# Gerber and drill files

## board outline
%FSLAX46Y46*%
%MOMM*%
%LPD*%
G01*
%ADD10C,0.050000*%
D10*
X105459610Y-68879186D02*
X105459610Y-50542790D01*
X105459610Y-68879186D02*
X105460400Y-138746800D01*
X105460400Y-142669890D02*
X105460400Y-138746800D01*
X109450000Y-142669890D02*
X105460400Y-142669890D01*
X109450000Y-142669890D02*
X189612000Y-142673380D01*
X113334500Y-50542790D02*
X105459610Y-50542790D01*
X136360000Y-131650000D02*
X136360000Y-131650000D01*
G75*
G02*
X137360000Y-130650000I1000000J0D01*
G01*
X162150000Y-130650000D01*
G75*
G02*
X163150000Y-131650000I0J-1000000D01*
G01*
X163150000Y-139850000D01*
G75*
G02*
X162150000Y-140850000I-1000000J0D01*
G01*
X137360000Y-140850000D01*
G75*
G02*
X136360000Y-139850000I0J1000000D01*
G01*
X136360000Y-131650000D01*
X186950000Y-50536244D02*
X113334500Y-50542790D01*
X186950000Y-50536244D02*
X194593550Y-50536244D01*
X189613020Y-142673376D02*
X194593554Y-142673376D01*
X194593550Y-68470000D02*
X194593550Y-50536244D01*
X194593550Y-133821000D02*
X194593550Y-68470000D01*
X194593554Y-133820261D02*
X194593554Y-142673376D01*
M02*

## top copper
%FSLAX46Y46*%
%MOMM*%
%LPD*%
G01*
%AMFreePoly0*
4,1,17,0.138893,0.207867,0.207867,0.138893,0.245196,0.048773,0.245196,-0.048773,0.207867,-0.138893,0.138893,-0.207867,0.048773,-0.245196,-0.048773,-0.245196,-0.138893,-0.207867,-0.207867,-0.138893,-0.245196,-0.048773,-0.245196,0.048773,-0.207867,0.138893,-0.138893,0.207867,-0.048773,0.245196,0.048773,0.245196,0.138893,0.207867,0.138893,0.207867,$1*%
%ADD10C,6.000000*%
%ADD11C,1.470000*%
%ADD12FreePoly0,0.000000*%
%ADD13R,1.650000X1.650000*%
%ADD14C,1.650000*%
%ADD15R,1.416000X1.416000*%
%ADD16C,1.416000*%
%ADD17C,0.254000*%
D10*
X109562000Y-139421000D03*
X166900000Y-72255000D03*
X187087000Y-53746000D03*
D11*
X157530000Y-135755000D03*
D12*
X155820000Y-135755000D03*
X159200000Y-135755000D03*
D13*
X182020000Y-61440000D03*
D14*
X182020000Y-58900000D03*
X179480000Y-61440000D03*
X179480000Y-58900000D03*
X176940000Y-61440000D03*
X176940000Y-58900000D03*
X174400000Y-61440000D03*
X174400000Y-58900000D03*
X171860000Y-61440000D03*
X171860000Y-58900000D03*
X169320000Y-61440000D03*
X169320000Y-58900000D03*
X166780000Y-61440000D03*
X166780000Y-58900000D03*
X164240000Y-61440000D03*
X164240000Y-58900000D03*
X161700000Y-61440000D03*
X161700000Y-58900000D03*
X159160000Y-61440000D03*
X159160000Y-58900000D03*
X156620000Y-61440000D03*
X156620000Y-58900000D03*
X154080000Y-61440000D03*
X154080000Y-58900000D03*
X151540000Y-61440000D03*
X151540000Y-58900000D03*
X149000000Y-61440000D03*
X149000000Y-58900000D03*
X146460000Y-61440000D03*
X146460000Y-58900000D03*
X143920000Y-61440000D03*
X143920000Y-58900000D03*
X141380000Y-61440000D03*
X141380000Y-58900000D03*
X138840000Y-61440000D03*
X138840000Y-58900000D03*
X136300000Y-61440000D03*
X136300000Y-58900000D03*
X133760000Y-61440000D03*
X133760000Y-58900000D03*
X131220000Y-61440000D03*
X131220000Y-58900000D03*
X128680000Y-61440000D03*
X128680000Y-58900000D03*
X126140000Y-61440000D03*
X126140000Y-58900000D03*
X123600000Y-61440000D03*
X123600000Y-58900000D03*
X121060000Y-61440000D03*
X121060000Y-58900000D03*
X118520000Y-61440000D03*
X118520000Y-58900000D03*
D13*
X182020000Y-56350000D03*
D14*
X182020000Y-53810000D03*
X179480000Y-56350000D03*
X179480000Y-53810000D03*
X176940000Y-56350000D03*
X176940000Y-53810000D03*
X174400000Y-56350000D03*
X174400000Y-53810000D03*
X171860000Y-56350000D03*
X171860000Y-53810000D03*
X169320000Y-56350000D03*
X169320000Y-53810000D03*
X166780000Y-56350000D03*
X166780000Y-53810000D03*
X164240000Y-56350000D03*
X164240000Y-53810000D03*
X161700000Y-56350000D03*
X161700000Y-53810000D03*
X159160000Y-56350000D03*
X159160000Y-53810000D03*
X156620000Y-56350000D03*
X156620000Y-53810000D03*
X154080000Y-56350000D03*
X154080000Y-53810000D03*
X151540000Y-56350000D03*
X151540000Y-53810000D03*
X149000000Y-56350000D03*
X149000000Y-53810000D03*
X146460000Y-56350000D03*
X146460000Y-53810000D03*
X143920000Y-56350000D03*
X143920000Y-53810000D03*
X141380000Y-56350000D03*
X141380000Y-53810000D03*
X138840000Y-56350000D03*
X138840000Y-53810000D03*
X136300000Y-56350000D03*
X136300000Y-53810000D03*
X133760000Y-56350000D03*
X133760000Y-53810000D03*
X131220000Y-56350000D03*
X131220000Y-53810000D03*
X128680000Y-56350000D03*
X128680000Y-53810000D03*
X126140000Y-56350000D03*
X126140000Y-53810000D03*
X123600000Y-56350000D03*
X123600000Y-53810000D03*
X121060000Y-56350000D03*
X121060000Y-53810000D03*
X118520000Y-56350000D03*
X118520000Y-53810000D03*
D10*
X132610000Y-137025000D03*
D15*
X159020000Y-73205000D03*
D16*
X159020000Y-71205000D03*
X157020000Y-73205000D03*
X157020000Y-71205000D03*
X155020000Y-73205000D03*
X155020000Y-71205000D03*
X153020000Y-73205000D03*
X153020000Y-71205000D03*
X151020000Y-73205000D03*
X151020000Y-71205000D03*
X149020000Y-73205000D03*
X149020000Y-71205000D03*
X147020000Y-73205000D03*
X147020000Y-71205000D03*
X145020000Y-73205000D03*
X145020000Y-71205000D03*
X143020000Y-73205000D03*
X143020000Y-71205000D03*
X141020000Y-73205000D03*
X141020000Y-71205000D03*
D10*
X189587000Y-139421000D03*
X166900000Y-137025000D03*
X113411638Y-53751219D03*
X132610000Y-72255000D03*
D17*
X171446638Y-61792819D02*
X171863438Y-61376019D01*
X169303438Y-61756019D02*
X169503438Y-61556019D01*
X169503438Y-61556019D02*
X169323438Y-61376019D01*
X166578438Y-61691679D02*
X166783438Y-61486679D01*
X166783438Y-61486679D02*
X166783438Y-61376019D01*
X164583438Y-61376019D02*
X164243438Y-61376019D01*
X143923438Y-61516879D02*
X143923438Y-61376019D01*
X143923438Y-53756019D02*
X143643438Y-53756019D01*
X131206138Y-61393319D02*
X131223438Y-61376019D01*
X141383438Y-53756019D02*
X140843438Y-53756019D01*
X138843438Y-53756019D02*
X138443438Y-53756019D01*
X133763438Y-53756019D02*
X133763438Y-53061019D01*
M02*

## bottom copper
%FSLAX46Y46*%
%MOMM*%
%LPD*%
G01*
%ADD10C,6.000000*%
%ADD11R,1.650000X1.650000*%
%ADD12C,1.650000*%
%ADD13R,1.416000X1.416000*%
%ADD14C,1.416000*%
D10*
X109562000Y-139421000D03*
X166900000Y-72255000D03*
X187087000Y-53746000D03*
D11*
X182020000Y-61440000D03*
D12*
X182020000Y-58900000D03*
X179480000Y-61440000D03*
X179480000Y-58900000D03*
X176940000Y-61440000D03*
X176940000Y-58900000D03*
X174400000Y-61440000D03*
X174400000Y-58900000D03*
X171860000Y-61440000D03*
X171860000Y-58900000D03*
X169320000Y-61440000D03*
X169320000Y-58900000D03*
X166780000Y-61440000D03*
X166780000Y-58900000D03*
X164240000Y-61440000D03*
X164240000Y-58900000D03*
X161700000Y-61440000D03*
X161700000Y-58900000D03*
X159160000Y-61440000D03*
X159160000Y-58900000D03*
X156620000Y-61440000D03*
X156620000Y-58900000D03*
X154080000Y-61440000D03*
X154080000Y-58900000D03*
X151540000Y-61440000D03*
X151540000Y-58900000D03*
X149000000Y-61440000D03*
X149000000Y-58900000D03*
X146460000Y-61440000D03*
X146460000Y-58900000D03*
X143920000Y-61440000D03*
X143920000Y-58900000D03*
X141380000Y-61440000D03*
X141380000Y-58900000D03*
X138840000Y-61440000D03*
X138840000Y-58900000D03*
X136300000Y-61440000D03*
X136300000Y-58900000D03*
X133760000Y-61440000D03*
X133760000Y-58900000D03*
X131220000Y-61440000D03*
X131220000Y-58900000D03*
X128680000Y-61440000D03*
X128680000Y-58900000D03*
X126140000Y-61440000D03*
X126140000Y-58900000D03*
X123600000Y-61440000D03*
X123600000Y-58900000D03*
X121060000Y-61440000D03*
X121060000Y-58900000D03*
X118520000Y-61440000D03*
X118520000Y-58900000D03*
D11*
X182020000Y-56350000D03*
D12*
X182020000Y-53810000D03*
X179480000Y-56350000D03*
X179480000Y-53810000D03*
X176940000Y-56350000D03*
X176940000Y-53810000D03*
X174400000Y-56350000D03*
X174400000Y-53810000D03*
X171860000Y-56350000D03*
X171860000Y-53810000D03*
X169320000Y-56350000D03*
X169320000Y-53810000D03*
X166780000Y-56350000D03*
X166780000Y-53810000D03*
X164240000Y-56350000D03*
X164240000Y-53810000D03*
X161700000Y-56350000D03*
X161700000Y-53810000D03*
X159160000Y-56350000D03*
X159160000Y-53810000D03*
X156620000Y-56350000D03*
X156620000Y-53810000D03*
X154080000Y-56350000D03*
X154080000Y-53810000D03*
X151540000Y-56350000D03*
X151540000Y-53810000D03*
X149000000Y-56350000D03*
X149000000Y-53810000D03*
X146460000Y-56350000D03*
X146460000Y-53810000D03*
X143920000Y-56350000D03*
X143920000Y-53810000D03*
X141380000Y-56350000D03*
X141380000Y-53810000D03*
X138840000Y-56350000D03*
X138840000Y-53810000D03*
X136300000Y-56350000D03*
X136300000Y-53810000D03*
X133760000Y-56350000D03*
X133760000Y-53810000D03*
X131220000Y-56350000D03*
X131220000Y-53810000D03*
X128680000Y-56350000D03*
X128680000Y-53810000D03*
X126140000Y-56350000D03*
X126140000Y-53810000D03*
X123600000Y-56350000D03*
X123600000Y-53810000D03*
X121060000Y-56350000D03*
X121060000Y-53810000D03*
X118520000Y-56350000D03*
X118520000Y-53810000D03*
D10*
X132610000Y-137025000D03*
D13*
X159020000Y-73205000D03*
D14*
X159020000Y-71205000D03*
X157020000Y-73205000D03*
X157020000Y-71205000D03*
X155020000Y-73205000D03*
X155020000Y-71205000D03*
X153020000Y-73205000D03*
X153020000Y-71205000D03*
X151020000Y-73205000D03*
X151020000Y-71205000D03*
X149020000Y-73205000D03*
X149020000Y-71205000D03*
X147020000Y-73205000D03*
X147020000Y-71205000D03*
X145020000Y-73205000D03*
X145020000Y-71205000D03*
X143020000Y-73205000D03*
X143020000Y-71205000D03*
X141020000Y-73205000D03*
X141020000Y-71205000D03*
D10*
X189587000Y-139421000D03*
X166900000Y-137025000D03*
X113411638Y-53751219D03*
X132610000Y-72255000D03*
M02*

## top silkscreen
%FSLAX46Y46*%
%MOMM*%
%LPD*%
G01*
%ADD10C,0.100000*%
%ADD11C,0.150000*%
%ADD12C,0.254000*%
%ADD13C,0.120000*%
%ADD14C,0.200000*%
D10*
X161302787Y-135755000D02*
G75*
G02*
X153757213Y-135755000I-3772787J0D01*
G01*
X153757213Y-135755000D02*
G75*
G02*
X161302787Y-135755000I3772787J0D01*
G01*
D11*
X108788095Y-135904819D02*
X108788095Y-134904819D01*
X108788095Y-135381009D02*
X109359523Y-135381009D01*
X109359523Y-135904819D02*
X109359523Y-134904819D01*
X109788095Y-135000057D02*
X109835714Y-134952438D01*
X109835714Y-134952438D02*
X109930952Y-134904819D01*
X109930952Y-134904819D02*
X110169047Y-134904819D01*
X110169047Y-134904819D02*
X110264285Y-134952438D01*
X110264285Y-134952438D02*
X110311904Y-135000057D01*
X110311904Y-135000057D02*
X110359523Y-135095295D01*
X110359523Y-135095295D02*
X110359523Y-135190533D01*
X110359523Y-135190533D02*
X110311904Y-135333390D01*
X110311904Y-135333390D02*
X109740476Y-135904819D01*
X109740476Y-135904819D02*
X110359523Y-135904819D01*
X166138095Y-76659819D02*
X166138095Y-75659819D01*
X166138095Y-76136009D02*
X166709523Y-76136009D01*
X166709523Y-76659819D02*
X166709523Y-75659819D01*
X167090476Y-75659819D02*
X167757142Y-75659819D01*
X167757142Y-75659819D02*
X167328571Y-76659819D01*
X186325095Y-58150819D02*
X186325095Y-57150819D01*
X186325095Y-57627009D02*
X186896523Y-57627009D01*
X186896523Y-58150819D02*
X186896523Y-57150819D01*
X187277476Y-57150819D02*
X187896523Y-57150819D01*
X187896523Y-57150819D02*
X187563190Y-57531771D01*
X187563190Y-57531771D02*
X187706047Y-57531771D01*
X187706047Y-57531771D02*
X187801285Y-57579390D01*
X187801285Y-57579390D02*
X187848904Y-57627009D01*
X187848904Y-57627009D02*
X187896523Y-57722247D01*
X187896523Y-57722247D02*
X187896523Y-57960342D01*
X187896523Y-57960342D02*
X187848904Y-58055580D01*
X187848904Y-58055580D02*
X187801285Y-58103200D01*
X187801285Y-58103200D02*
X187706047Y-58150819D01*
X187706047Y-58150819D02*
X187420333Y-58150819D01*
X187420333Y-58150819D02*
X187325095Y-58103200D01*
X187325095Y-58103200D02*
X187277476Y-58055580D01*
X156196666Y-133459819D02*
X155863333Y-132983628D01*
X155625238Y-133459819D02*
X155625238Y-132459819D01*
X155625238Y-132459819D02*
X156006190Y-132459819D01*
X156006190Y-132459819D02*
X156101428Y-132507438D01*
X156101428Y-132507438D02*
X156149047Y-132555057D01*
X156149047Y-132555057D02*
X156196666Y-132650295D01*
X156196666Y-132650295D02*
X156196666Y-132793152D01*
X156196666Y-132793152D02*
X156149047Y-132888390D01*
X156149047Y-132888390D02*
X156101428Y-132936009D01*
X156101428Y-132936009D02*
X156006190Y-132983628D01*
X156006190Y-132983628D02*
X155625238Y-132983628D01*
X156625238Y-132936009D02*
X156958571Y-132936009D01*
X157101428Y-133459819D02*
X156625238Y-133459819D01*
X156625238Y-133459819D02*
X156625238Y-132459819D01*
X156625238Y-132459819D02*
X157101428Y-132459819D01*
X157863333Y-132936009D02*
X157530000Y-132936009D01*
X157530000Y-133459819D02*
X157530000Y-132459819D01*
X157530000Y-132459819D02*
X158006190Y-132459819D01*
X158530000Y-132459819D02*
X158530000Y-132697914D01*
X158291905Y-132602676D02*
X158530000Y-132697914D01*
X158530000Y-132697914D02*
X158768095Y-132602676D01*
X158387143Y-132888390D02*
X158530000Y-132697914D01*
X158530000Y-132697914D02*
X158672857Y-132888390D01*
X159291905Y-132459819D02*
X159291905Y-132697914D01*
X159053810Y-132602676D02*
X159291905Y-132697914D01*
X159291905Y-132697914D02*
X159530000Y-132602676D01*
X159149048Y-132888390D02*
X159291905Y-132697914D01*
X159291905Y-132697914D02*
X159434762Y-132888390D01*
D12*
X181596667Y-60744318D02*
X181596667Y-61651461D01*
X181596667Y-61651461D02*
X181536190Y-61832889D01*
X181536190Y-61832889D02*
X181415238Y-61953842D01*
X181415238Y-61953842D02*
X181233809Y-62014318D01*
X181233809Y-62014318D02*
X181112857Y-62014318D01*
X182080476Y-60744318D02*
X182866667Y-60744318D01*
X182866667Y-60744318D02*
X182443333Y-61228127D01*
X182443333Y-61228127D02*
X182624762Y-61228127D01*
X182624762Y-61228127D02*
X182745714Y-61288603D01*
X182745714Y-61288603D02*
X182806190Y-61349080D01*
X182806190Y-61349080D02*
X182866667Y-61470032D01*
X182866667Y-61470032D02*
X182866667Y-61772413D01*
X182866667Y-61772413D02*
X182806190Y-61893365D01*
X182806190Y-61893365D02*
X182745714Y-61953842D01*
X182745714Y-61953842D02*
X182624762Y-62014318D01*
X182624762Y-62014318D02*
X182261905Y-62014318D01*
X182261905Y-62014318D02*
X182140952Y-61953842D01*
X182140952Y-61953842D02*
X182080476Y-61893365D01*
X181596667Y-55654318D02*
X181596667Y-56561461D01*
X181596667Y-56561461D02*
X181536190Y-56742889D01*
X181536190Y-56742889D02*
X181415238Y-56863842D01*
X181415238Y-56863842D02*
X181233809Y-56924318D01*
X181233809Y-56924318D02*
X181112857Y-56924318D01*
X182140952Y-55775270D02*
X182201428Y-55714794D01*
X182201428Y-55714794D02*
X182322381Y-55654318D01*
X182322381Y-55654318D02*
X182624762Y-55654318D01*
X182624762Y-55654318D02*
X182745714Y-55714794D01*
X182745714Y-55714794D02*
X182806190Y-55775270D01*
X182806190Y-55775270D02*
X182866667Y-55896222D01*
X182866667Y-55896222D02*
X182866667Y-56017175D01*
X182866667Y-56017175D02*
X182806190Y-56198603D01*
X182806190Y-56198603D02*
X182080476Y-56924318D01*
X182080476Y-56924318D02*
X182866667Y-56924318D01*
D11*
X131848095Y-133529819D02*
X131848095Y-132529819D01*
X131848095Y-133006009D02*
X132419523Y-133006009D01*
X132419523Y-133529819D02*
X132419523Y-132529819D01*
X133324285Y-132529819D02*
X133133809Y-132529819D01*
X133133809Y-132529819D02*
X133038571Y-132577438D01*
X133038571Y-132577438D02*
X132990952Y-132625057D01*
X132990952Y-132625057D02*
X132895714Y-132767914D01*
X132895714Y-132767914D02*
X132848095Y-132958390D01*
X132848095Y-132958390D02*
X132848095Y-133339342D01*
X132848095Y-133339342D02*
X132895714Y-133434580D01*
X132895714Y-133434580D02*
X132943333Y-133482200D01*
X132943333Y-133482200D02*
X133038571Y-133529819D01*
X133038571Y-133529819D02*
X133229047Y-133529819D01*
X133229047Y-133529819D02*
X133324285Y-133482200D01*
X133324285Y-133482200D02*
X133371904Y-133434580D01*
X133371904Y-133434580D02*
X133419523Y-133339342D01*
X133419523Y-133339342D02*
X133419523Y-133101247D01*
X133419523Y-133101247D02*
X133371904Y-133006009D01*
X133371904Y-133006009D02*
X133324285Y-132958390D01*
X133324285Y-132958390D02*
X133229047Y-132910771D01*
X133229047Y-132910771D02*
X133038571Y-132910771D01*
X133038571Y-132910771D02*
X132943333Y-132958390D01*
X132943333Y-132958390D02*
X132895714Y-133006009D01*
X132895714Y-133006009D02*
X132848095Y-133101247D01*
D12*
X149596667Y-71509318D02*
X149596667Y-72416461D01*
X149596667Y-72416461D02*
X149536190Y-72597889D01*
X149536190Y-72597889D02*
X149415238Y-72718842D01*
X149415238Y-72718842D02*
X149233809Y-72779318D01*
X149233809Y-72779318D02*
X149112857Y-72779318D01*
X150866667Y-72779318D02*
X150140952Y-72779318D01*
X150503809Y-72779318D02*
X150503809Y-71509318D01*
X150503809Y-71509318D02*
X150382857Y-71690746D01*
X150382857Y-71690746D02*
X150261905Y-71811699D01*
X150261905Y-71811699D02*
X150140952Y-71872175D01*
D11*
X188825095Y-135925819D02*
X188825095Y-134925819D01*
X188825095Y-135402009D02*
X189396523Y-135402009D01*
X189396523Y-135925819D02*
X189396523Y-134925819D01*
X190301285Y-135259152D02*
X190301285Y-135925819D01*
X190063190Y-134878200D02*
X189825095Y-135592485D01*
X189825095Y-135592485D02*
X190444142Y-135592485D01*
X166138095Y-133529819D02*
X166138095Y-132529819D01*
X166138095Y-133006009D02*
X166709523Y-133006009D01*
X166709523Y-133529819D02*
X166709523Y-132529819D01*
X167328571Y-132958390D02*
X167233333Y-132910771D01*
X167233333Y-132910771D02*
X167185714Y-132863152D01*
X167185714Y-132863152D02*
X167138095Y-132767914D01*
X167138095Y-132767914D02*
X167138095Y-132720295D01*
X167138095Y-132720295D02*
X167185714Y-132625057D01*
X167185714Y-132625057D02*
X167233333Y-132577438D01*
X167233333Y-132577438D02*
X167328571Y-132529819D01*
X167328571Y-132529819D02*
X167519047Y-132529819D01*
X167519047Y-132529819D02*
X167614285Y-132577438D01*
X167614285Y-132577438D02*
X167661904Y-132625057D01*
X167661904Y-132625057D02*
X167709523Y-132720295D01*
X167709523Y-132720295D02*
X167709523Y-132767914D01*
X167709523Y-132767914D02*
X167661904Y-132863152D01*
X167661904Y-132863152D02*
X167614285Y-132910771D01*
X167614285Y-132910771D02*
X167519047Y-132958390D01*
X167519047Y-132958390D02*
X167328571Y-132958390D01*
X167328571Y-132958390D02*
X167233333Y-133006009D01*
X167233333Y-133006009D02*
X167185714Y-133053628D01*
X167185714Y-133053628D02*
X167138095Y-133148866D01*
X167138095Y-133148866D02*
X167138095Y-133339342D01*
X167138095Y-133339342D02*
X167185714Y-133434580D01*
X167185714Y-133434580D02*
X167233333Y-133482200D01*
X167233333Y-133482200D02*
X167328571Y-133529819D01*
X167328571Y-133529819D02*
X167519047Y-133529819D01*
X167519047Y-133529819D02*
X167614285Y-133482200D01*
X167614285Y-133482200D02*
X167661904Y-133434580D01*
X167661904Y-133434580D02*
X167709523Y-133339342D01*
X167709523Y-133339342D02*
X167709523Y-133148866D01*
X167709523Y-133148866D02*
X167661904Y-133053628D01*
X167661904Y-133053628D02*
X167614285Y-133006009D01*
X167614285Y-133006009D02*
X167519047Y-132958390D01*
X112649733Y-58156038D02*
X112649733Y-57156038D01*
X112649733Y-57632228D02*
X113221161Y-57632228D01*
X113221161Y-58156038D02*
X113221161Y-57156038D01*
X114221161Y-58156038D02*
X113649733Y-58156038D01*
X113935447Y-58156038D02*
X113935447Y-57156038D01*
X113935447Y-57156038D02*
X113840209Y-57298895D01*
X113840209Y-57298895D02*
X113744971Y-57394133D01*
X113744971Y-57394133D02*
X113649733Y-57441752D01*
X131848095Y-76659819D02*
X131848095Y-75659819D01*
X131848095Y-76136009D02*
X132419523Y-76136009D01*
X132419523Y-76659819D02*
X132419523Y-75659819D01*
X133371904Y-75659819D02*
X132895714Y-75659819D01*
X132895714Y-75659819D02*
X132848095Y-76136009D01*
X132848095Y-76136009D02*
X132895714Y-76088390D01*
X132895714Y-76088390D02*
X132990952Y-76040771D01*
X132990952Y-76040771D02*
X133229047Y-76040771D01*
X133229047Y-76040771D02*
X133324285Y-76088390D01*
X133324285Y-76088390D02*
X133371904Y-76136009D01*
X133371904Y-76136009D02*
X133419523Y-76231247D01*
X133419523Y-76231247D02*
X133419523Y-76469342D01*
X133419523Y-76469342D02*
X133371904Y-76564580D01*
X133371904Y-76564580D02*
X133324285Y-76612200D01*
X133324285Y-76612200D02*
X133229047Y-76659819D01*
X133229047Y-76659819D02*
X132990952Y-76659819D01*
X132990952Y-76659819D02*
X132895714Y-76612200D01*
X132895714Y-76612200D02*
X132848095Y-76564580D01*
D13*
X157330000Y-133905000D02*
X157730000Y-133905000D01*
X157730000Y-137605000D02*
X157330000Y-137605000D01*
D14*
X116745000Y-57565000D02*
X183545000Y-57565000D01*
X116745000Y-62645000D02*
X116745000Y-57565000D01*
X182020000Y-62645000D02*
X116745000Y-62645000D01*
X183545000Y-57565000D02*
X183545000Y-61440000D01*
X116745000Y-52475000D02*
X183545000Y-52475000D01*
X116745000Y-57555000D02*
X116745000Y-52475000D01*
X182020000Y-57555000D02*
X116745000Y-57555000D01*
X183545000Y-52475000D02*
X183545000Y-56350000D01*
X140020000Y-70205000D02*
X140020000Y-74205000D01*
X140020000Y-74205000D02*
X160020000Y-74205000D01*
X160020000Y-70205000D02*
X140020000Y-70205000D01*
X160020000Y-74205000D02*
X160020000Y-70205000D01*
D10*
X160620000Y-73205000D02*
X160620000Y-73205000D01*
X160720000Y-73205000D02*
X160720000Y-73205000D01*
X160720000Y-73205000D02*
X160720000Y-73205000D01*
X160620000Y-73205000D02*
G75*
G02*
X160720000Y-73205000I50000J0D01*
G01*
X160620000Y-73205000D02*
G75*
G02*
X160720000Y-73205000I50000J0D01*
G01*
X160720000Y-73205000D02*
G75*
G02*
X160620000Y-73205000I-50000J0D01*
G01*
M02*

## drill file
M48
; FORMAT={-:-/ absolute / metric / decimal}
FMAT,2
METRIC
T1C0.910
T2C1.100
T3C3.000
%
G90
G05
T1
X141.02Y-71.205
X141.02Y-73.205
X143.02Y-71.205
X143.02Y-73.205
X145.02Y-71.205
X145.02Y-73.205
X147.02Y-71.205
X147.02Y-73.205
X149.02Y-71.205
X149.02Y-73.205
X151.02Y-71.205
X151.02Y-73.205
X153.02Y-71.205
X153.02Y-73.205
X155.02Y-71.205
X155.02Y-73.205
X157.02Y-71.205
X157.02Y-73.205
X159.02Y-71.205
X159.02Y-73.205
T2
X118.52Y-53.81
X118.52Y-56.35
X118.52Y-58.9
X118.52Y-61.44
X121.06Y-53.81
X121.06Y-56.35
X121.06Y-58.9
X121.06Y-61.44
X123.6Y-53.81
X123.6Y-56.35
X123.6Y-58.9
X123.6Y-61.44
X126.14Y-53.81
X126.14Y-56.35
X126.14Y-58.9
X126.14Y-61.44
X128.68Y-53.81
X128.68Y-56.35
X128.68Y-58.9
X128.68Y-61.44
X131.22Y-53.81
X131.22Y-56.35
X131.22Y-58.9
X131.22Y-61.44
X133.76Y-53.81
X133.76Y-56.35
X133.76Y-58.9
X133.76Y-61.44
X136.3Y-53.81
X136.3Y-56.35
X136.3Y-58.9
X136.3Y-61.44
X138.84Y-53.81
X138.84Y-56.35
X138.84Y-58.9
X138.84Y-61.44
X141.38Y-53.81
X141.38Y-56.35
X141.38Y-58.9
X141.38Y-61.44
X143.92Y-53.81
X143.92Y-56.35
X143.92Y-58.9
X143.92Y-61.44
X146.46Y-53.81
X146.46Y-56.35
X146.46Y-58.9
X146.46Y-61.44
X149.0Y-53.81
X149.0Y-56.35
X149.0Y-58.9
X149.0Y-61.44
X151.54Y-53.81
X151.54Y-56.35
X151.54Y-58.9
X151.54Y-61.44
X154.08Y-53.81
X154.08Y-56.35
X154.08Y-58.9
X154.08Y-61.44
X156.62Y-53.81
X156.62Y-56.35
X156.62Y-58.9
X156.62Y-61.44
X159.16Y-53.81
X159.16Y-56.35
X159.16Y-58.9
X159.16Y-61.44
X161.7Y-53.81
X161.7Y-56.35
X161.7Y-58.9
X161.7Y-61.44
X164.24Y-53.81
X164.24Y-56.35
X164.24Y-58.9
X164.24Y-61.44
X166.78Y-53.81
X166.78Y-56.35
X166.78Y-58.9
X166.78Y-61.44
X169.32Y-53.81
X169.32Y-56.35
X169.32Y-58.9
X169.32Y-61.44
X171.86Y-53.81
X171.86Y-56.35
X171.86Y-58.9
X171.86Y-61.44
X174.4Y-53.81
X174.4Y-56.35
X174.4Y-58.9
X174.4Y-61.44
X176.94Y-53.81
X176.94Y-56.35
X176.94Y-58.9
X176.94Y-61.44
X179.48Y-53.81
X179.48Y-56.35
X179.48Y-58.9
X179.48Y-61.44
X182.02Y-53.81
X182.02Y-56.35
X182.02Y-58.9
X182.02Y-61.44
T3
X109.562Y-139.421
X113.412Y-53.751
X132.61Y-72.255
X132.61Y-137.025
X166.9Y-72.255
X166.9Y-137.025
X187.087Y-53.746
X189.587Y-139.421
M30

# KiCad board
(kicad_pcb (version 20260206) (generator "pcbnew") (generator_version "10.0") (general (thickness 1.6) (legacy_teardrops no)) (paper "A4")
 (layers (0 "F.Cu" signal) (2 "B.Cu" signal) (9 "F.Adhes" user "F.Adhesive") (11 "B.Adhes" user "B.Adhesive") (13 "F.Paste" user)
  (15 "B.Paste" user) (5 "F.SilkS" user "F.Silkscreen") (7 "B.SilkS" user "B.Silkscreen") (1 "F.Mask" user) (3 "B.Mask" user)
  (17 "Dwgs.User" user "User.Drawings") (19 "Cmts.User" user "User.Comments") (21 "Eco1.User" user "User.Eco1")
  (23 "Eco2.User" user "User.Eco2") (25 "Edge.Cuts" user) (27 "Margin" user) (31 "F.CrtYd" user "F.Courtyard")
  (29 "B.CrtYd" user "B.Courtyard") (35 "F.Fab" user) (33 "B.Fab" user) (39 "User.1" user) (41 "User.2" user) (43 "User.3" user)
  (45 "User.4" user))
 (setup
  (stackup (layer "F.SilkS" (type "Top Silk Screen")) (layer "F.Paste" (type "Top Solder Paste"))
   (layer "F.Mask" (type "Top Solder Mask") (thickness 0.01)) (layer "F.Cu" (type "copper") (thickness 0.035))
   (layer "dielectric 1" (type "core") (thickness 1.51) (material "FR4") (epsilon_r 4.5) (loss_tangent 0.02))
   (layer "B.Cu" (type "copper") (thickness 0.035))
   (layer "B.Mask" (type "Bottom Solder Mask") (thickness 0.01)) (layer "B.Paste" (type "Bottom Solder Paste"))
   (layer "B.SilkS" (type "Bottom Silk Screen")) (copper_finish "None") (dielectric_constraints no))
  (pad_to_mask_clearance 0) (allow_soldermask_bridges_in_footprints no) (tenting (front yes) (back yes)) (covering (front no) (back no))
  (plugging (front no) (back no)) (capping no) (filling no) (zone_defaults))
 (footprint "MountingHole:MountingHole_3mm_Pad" (layer "F.Cu") (at 109.562 139.421 180)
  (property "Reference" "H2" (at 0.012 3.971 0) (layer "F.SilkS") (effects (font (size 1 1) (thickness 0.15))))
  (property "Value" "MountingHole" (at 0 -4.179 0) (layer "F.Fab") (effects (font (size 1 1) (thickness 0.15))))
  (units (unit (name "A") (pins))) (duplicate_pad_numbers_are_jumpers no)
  (pad "1" thru_hole circle (at 0 0 180) (size 6 6) (drill 3) (layers "*.Cu" "*.Mask") (remove_unused_layers no) (zone_connect 2)))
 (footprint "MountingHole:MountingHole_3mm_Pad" (layer "F.Cu") (at 166.9 72.255)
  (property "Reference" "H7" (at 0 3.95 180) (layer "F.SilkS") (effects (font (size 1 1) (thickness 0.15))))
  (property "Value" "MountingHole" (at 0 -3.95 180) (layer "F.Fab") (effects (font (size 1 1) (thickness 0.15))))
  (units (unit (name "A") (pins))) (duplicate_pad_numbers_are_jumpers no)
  (pad "1" thru_hole circle (at 0 0) (size 6 6) (drill 3) (layers "*.Cu" "*.Mask") (remove_unused_layers no) (zone_connect 2)))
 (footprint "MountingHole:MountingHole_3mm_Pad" (layer "F.Cu") (at 187.087 53.746 180)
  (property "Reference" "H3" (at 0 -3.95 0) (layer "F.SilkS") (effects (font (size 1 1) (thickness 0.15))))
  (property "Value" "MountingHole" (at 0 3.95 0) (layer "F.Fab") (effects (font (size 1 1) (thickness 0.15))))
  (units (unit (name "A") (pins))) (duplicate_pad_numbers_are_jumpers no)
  (pad "1" thru_hole circle (at 0 0 180) (size 6 6) (drill 3) (layers "*.Cu" "*.Mask") (remove_unused_layers no) (zone_connect 2)))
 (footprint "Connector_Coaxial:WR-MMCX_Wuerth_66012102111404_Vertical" (layer "F.Cu") (at 157.53 135.755)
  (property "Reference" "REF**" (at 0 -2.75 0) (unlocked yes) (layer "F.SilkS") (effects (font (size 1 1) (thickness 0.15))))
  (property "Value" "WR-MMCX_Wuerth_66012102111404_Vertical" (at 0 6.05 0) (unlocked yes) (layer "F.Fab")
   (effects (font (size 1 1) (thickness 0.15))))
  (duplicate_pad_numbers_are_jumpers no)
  (fp_line (start -0.2 -1.85) (end 0.2 -1.85) (stroke (width 0.12) (type solid)) (layer "F.SilkS"))
  (fp_line (start 0.2 1.85) (end -0.2 1.85) (stroke (width 0.12) (type solid)) (layer "F.SilkS"))
  (pad "1" smd circle (at 0 0) (size 1.47 1.47) (layers "F.Cu" "F.Mask" "F.Paste"))
  (pad "2" smd custom (at -1.71 0) (size 0.5 0.5) (layers "F.Cu" "F.Mask") (options (clearance outline) (anchor circle)) (primitives))
  (pad "2" smd custom (at 1.67 0) (size 0.5 0.5) (layers "F.Cu" "F.Mask") (options (clearance outline) (anchor circle)) (primitives)))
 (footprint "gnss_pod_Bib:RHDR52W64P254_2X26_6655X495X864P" (layer "F.Cu") (at 182.02 61.44)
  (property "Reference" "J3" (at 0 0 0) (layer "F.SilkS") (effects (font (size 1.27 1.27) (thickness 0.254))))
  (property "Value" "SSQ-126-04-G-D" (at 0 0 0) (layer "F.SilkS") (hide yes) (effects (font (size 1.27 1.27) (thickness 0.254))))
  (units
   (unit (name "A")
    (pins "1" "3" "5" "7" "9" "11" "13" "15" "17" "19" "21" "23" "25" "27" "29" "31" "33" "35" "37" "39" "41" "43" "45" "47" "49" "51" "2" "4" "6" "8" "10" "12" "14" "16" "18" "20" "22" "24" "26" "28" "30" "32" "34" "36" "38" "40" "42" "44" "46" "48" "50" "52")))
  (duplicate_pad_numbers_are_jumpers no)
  (fp_line (start -65.275 -3.875) (end 1.525 -3.875) (stroke (width 0.2) (type solid)) (layer "F.SilkS"))
  (fp_line (start -65.275 1.205) (end -65.275 -3.875) (stroke (width 0.2) (type solid)) (layer "F.SilkS"))
  (fp_line (start 0 1.205) (end -65.275 1.205) (stroke (width 0.2) (type solid)) (layer "F.SilkS"))
  (fp_line (start 1.525 -3.875) (end 1.525 0) (stroke (width 0.2) (type solid)) (layer "F.SilkS"))
  (pad "1" thru_hole rect (at 0 0) (size 1.65 1.65) (drill 1.1) (layers "*.Cu" "*.Mask") (remove_unused_layers no)
   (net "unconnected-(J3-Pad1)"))
  (pad "2" thru_hole circle (at 0 -2.54) (size 1.65 1.65) (drill 1.1) (layers "*.Cu" "*.Mask") (remove_unused_layers no)
   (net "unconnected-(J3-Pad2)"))
  (pad "3" thru_hole circle (at -2.54 0) (size 1.65 1.65) (drill 1.1) (layers "*.Cu" "*.Mask") (remove_unused_layers no)
   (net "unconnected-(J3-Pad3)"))
  (pad "4" thru_hole circle (at -2.54 -2.54) (size 1.65 1.65) (drill 1.1) (layers "*.Cu" "*.Mask") (remove_unused_layers no)
   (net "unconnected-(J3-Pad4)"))
  (pad "5" thru_hole circle (at -5.08 0) (size 1.65 1.65) (drill 1.1) (layers "*.Cu" "*.Mask") (remove_unused_layers no)
   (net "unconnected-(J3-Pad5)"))
  (pad "6" thru_hole circle (at -5.08 -2.54) (size 1.65 1.65) (drill 1.1) (layers "*.Cu" "*.Mask") (remove_unused_layers no)
   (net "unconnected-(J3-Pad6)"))
  (pad "7" thru_hole circle (at -7.62 0) (size 1.65 1.65) (drill 1.1) (layers "*.Cu" "*.Mask") (remove_unused_layers no)
   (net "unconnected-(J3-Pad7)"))
  (pad "8" thru_hole circle (at -7.62 -2.54) (size 1.65 1.65) (drill 1.1) (layers "*.Cu" "*.Mask") (remove_unused_layers no)
   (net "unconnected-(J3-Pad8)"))
  (pad "9" thru_hole circle (at -10.16 0) (size 1.65 1.65) (drill 1.1) (layers "*.Cu" "*.Mask") (remove_unused_layers no)
   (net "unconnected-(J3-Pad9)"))
  (pad "10" thru_hole circle (at -10.16 -2.54) (size 1.65 1.65) (drill 1.1) (layers "*.Cu" "*.Mask") (remove_unused_layers no)
   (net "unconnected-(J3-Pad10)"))
  (pad "11" thru_hole circle (at -12.7 0) (size 1.65 1.65) (drill 1.1) (layers "*.Cu" "*.Mask") (remove_unused_layers no)
   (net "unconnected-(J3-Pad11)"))
  (pad "12" thru_hole circle (at -12.7 -2.54) (size 1.65 1.65) (drill 1.1) (layers "*.Cu" "*.Mask") (remove_unused_layers no)
   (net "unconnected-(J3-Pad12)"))
  (pad "13" thru_hole circle (at -15.24 0) (size 1.65 1.65) (drill 1.1) (layers "*.Cu" "*.Mask") (remove_unused_layers no)
   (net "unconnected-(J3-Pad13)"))
  (pad "14" thru_hole circle (at -15.24 -2.54) (size 1.65 1.65) (drill 1.1) (layers "*.Cu" "*.Mask") (remove_unused_layers no)
   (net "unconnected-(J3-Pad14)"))
  (pad "15" thru_hole circle (at -17.78 0) (size 1.65 1.65) (drill 1.1) (layers "*.Cu" "*.Mask") (remove_unused_layers no)
   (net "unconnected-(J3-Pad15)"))
  (pad "16" thru_hole circle (at -17.78 -2.54) (size 1.65 1.65) (drill 1.1) (layers "*.Cu" "*.Mask") (remove_unused_layers no)
   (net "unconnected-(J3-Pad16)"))
  (pad "17" thru_hole circle (at -20.32 0) (size 1.65 1.65) (drill 1.1) (layers "*.Cu" "*.Mask") (remove_unused_layers no)
   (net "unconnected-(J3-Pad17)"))
  (pad "18" thru_hole circle (at -20.32 -2.54) (size 1.65 1.65) (drill 1.1) (layers "*.Cu" "*.Mask") (remove_unused_layers no)
   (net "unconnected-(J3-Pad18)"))
  (pad "19" thru_hole circle (at -22.86 0) (size 1.65 1.65) (drill 1.1) (layers "*.Cu" "*.Mask") (remove_unused_layers no)
   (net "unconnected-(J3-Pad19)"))
  (pad "20" thru_hole circle (at -22.86 -2.54) (size 1.65 1.65) (drill 1.1) (layers "*.Cu" "*.Mask") (remove_unused_layers no)
   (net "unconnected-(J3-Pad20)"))
  (pad "21" thru_hole circle (at -25.4 0) (size 1.65 1.65) (drill 1.1) (layers "*.Cu" "*.Mask") (remove_unused_layers no)
   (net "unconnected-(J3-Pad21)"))
  (pad "22" thru_hole circle (at -25.4 -2.54) (size 1.65 1.65) (drill 1.1) (layers "*.Cu" "*.Mask") (remove_unused_layers no)
   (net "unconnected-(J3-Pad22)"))
  (pad "23" thru_hole circle (at -27.94 0) (size 1.65 1.65) (drill 1.1) (layers "*.Cu" "*.Mask") (remove_unused_layers no)
   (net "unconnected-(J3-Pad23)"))
  (pad "24" thru_hole circle (at -27.94 -2.54) (size 1.65 1.65) (drill 1.1) (layers "*.Cu" "*.Mask") (remove_unused_layers no)
   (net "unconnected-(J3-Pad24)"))
  (pad "25" thru_hole circle (at -30.48 0) (size 1.65 1.65) (drill 1.1) (layers "*.Cu" "*.Mask") (remove_unused_layers no)
   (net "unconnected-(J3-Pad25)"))
  (pad "26" thru_hole circle (at -30.48 -2.54) (size 1.65 1.65) (drill 1.1) (layers "*.Cu" "*.Mask") (remove_unused_layers no)
   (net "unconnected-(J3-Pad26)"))
  (pad "27" thru_hole circle (at -33.02 0) (size 1.65 1.65) (drill 1.1) (layers "*.Cu" "*.Mask") (remove_unused_layers no)
   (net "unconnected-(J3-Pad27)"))
  (pad "28" thru_hole circle (at -33.02 -2.54) (size 1.65 1.65) (drill 1.1) (layers "*.Cu" "*.Mask") (remove_unused_layers no)
   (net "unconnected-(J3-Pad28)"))
  (pad "29" thru_hole circle (at -35.56 0) (size 1.65 1.65) (drill 1.1) (layers "*.Cu" "*.Mask") (remove_unused_layers no) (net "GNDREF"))
  (pad "30" thru_hole circle (at -35.56 -2.54) (size 1.65 1.65) (drill 1.1) (layers "*.Cu" "*.Mask") (remove_unused_layers no)
   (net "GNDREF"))
  (pad "31" thru_hole circle (at -38.1 0) (size 1.65 1.65) (drill 1.1) (layers "*.Cu" "*.Mask") (remove_unused_layers no) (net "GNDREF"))
  (pad "32" thru_hole circle (at -38.1 -2.54) (size 1.65 1.65) (drill 1.1) (layers "*.Cu" "*.Mask") (remove_unused_layers no) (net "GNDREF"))
  (pad "33" thru_hole circle (at -40.64 0) (size 1.65 1.65) (drill 1.1) (layers "*.Cu" "*.Mask") (remove_unused_layers no)
   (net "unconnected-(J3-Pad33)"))
  (pad "34" thru_hole circle (at -40.64 -2.54) (size 1.65 1.65) (drill 1.1) (layers "*.Cu" "*.Mask") (remove_unused_layers no)
   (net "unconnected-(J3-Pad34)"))
  (pad "35" thru_hole circle (at -43.18 0) (size 1.65 1.65) (drill 1.1) (layers "*.Cu" "*.Mask") (remove_unused_layers no)
   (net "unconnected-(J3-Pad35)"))
  (pad "36" thru_hole circle (at -43.18 -2.54) (size 1.65 1.65) (drill 1.1) (layers "*.Cu" "*.Mask") (remove_unused_layers no)
   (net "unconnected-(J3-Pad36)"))
  (pad "37" thru_hole circle (at -45.72 0) (size 1.65 1.65) (drill 1.1) (layers "*.Cu" "*.Mask") (remove_unused_layers no)
   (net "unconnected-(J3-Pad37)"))
  (pad "38" thru_hole circle (at -45.72 -2.54) (size 1.65 1.65) (drill 1.1) (layers "*.Cu" "*.Mask") (remove_unused_layers no)
   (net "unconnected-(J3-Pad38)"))
  (pad "39" thru_hole circle (at -48.26 0) (size 1.65 1.65) (drill 1.1) (layers "*.Cu" "*.Mask") (remove_unused_layers no)
   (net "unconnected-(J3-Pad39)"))
  (pad "40" thru_hole circle (at -48.26 -2.54) (size 1.65 1.65) (drill 1.1) (layers "*.Cu" "*.Mask") (remove_unused_layers no)
   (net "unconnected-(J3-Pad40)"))
  (pad "41" thru_hole circle (at -50.8 0) (size 1.65 1.65) (drill 1.1) (layers "*.Cu" "*.Mask") (remove_unused_layers no)
   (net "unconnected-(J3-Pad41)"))
  (pad "42" thru_hole circle (at -50.8 -2.54) (size 1.65 1.65) (drill 1.1) (layers "*.Cu" "*.Mask") (remove_unused_layers no)
   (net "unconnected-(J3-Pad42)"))
  (pad "43" thru_hole circle (at -53.34 0) (size 1.65 1.65) (drill 1.1) (layers "*.Cu" "*.Mask") (remove_unused_layers no)
   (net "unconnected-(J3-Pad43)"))
  (pad "44" thru_hole circle (at -53.34 -2.54) (size 1.65 1.65) (drill 1.1) (layers "*.Cu" "*.Mask") (remove_unused_layers no)
   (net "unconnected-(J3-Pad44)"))
  (pad "45" thru_hole circle (at -55.88 0) (size 1.65 1.65) (drill 1.1) (layers "*.Cu" "*.Mask") (remove_unused_layers no)
   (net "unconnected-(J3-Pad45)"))
  (pad "46" thru_hole circle (at -55.88 -2.54) (size 1.65 1.65) (drill 1.1) (layers "*.Cu" "*.Mask") (remove_unused_layers no)
   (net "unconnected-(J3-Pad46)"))
  (pad "47" thru_hole circle (at -58.42 0) (size 1.65 1.65) (drill 1.1) (layers "*.Cu" "*.Mask") (remove_unused_layers no)
   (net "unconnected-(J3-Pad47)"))
  (pad "48" thru_hole circle (at -58.42 -2.54) (size 1.65 1.65) (drill 1.1) (layers "*.Cu" "*.Mask") (remove_unused_layers no)
   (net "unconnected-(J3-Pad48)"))
  (pad "49" thru_hole circle (at -60.96 0) (size 1.65 1.65) (drill 1.1) (layers "*.Cu" "*.Mask") (remove_unused_layers no)
   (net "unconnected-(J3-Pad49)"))
  (pad "50" thru_hole circle (at -60.96 -2.54) (size 1.65 1.65) (drill 1.1) (layers "*.Cu" "*.Mask") (remove_unused_layers no)
   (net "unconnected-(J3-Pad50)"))
  (pad "51" thru_hole circle (at -63.5 0) (size 1.65 1.65) (drill 1.1) (layers "*.Cu" "*.Mask") (remove_unused_layers no)
   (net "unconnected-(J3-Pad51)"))
  (pad "52" thru_hole circle (at -63.5 -2.54) (size 1.65 1.65) (drill 1.1) (layers "*.Cu" "*.Mask") (remove_unused_layers no)
   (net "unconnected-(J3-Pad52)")))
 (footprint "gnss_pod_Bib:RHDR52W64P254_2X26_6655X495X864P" (layer "F.Cu") (at 182.02 56.35)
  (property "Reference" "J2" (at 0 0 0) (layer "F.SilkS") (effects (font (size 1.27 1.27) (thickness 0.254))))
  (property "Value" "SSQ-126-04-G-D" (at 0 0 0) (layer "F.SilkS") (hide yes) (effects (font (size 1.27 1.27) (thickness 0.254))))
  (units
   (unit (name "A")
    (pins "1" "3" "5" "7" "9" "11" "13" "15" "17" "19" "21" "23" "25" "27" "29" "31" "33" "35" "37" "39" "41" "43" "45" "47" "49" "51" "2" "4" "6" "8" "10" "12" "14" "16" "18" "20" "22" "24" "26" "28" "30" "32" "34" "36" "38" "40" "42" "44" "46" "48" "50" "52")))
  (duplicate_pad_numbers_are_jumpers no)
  (fp_line (start -65.275 -3.875) (end 1.525 -3.875) (stroke (width 0.2) (type solid)) (layer "F.SilkS"))
  (fp_line (start -65.275 1.205) (end -65.275 -3.875) (stroke (width 0.2) (type solid)) (layer "F.SilkS"))
  (fp_line (start 0 1.205) (end -65.275 1.205) (stroke (width 0.2) (type solid)) (layer "F.SilkS"))
  (fp_line (start 1.525 -3.875) (end 1.525 0) (stroke (width 0.2) (type solid)) (layer "F.SilkS"))
  (pad "1" thru_hole rect (at 0 0) (size 1.65 1.65) (drill 1.1) (layers "*.Cu" "*.Mask") (remove_unused_layers no)
   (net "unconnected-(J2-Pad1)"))
  (pad "2" thru_hole circle (at 0 -2.54) (size 1.65 1.65) (drill 1.1) (layers "*.Cu" "*.Mask") (remove_unused_layers no)
   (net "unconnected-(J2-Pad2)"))
  (pad "3" thru_hole circle (at -2.54 0) (size 1.65 1.65) (drill 1.1) (layers "*.Cu" "*.Mask") (remove_unused_layers no)
   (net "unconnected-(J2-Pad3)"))
  (pad "4" thru_hole circle (at -2.54 -2.54) (size 1.65 1.65) (drill 1.1) (layers "*.Cu" "*.Mask") (remove_unused_layers no)
   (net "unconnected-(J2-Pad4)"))
  (pad "5" thru_hole circle (at -5.08 0) (size 1.65 1.65) (drill 1.1) (layers "*.Cu" "*.Mask") (remove_unused_layers no)
   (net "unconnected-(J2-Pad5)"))
  (pad "6" thru_hole circle (at -5.08 -2.54) (size 1.65 1.65) (drill 1.1) (layers "*.Cu" "*.Mask") (remove_unused_layers no)
   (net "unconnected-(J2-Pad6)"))
  (pad "7" thru_hole circle (at -7.62 0) (size 1.65 1.65) (drill 1.1) (layers "*.Cu" "*.Mask") (remove_unused_layers no)
   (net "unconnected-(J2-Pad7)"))
  (pad "8" thru_hole circle (at -7.62 -2.54) (size 1.65 1.65) (drill 1.1) (layers "*.Cu" "*.Mask") (remove_unused_layers no)
   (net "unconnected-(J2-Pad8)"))
  (pad "9" thru_hole circle (at -10.16 0) (size 1.65 1.65) (drill 1.1) (layers "*.Cu" "*.Mask") (remove_unused_layers no)
   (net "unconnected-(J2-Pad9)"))
  (pad "10" thru_hole circle (at -10.16 -2.54) (size 1.65 1.65) (drill 1.1) (layers "*.Cu" "*.Mask") (remove_unused_layers no)
   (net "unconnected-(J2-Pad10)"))
  (pad "11" thru_hole circle (at -12.7 0) (size 1.65 1.65) (drill 1.1) (layers "*.Cu" "*.Mask") (remove_unused_layers no)
   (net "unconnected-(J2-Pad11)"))
  (pad "12" thru_hole circle (at -12.7 -2.54) (size 1.65 1.65) (drill 1.1) (layers "*.Cu" "*.Mask") (remove_unused_layers no)
   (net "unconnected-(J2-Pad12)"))
  (pad "13" thru_hole circle (at -15.24 0) (size 1.65 1.65) (drill 1.1) (layers "*.Cu" "*.Mask") (remove_unused_layers no)
   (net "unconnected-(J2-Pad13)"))
  (pad "14" thru_hole circle (at -15.24 -2.54) (size 1.65 1.65) (drill 1.1) (layers "*.Cu" "*.Mask") (remove_unused_layers no)
   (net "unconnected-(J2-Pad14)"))
  (pad "15" thru_hole circle (at -17.78 0) (size 1.65 1.65) (drill 1.1) (layers "*.Cu" "*.Mask") (remove_unused_layers no)
   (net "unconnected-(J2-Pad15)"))
  (pad "16" thru_hole circle (at -17.78 -2.54) (size 1.65 1.65) (drill 1.1) (layers "*.Cu" "*.Mask") (remove_unused_layers no)
   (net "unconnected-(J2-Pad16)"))
  (pad "17" thru_hole circle (at -20.32 0) (size 1.65 1.65) (drill 1.1) (layers "*.Cu" "*.Mask") (remove_unused_layers no) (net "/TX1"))
  (pad "18" thru_hole circle (at -20.32 -2.54) (size 1.65 1.65) (drill 1.1) (layers "*.Cu" "*.Mask") (remove_unused_layers no)
   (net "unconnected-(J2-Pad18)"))
  (pad "19" thru_hole circle (at -22.86 0) (size 1.65 1.65) (drill 1.1) (layers "*.Cu" "*.Mask") (remove_unused_layers no) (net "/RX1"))
  (pad "20" thru_hole circle (at -22.86 -2.54) (size 1.65 1.65) (drill 1.1) (layers "*.Cu" "*.Mask") (remove_unused_layers no)
   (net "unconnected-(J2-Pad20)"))
  (pad "21" thru_hole circle (at -25.4 0) (size 1.65 1.65) (drill 1.1) (layers "*.Cu" "*.Mask") (remove_unused_layers no)
   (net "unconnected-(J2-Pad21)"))
  (pad "22" thru_hole circle (at -25.4 -2.54) (size 1.65 1.65) (drill 1.1) (layers "*.Cu" "*.Mask") (remove_unused_layers no)
   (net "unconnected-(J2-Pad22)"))
  (pad "23" thru_hole circle (at -27.94 0) (size 1.65 1.65) (drill 1.1) (layers "*.Cu" "*.Mask") (remove_unused_layers no)
   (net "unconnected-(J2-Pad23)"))
  (pad "24" thru_hole circle (at -27.94 -2.54) (size 1.65 1.65) (drill 1.1) (layers "*.Cu" "*.Mask") (remove_unused_layers no)
   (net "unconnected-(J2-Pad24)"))
  (pad "25" thru_hole circle (at -30.48 0) (size 1.65 1.65) (drill 1.1) (layers "*.Cu" "*.Mask") (remove_unused_layers no)
   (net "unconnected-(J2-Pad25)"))
  (pad "26" thru_hole circle (at -30.48 -2.54) (size 1.65 1.65) (drill 1.1) (layers "*.Cu" "*.Mask") (remove_unused_layers no)
   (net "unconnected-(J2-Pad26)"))
  (pad "27" thru_hole circle (at -33.02 0) (size 1.65 1.65) (drill 1.1) (layers "*.Cu" "*.Mask") (remove_unused_layers no)
   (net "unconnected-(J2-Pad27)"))
  (pad "28" thru_hole circle (at -33.02 -2.54) (size 1.65 1.65) (drill 1.1) (layers "*.Cu" "*.Mask") (remove_unused_layers no)
   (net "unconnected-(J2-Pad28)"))
  (pad "29" thru_hole circle (at -35.56 0) (size 1.65 1.65) (drill 1.1) (layers "*.Cu" "*.Mask") (remove_unused_layers no) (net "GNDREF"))
  (pad "30" thru_hole circle (at -35.56 -2.54) (size 1.65 1.65) (drill 1.1) (layers "*.Cu" "*.Mask") (remove_unused_layers no)
   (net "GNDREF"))
  (pad "31" thru_hole circle (at -38.1 0) (size 1.65 1.65) (drill 1.1) (layers "*.Cu" "*.Mask") (remove_unused_layers no) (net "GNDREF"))
  (pad "32" thru_hole circle (at -38.1 -2.54) (size 1.65 1.65) (drill 1.1) (layers "*.Cu" "*.Mask") (remove_unused_layers no) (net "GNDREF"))
  (pad "33" thru_hole circle (at -40.64 0) (size 1.65 1.65) (drill 1.1) (layers "*.Cu" "*.Mask") (remove_unused_layers no)
   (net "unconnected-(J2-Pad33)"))
  (pad "34" thru_hole circle (at -40.64 -2.54) (size 1.65 1.65) (drill 1.1) (layers "*.Cu" "*.Mask") (remove_unused_layers no)
   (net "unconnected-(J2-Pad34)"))
  (pad "35" thru_hole circle (at -43.18 0) (size 1.65 1.65) (drill 1.1) (layers "*.Cu" "*.Mask") (remove_unused_layers no)
   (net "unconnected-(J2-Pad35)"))
  (pad "36" thru_hole circle (at -43.18 -2.54) (size 1.65 1.65) (drill 1.1) (layers "*.Cu" "*.Mask") (remove_unused_layers no)
   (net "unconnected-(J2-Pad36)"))
  (pad "37" thru_hole circle (at -45.72 0) (size 1.65 1.65) (drill 1.1) (layers "*.Cu" "*.Mask") (remove_unused_layers no)
   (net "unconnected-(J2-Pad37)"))
  (pad "38" thru_hole circle (at -45.72 -2.54) (size 1.65 1.65) (drill 1.1) (layers "*.Cu" "*.Mask") (remove_unused_layers no)
   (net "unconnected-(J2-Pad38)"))
  (pad "39" thru_hole circle (at -48.26 0) (size 1.65 1.65) (drill 1.1) (layers "*.Cu" "*.Mask") (remove_unused_layers no)
   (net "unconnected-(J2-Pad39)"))
  (pad "40" thru_hole circle (at -48.26 -2.54) (size 1.65 1.65) (drill 1.1) (layers "*.Cu" "*.Mask") (remove_unused_layers no)
   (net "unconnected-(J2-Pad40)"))
  (pad "41" thru_hole circle (at -50.8 0) (size 1.65 1.65) (drill 1.1) (layers "*.Cu" "*.Mask") (remove_unused_layers no)
   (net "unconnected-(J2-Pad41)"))
  (pad "42" thru_hole circle (at -50.8 -2.54) (size 1.65 1.65) (drill 1.1) (layers "*.Cu" "*.Mask") (remove_unused_layers no)
   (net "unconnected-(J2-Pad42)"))
  (pad "43" thru_hole circle (at -53.34 0) (size 1.65 1.65) (drill 1.1) (layers "*.Cu" "*.Mask") (remove_unused_layers no)
   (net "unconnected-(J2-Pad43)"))
  (pad "44" thru_hole circle (at -53.34 -2.54) (size 1.65 1.65) (drill 1.1) (layers "*.Cu" "*.Mask") (remove_unused_layers no)
   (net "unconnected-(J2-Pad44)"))
  (pad "45" thru_hole circle (at -55.88 0) (size 1.65 1.65) (drill 1.1) (layers "*.Cu" "*.Mask") (remove_unused_layers no)
   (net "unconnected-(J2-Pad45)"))
  (pad "46" thru_hole circle (at -55.88 -2.54) (size 1.65 1.65) (drill 1.1) (layers "*.Cu" "*.Mask") (remove_unused_layers no)
   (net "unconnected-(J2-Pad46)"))
  (pad "47" thru_hole circle (at -58.42 0) (size 1.65 1.65) (drill 1.1) (layers "*.Cu" "*.Mask") (remove_unused_layers no)
   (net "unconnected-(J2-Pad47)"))
  (pad "48" thru_hole circle (at -58.42 -2.54) (size 1.65 1.65) (drill 1.1) (layers "*.Cu" "*.Mask") (remove_unused_layers no)
   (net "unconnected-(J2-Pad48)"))
  (pad "49" thru_hole circle (at -60.96 0) (size 1.65 1.65) (drill 1.1) (layers "*.Cu" "*.Mask") (remove_unused_layers no)
   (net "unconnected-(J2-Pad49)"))
  (pad "50" thru_hole circle (at -60.96 -2.54) (size 1.65 1.65) (drill 1.1) (layers "*.Cu" "*.Mask") (remove_unused_layers no)
   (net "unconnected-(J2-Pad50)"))
  (pad "51" thru_hole circle (at -63.5 0) (size 1.65 1.65) (drill 1.1) (layers "*.Cu" "*.Mask") (remove_unused_layers no)
   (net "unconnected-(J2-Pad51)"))
  (pad "52" thru_hole circle (at -63.5 -2.54) (size 1.65 1.65) (drill 1.1) (layers "*.Cu" "*.Mask") (remove_unused_layers no)
   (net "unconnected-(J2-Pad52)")))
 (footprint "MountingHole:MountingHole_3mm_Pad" (layer "F.Cu") (at 132.61 137.025)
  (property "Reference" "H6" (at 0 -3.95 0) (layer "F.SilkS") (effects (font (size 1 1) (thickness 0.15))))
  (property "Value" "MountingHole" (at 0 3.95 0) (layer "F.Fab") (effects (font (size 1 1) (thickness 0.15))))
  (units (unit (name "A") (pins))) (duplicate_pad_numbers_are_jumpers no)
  (pad "1" thru_hole circle (at 0 0) (size 6 6) (drill 3) (layers "*.Cu" "*.Mask") (remove_unused_layers no) (zone_connect 2)))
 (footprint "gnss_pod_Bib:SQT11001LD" (layer "F.Cu") (at 159.02 73.205)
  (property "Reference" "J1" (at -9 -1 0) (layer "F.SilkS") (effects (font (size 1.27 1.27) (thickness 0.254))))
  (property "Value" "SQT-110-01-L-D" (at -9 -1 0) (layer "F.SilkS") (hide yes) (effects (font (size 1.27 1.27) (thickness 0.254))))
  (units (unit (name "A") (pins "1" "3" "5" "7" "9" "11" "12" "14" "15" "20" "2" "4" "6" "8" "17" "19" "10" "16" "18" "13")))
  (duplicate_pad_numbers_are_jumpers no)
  (fp_line (start -19 -3) (end -19 1) (stroke (width 0.2) (type solid)) (layer "F.SilkS"))
  (fp_line (start -19 1) (end 1 1) (stroke (width 0.2) (type solid)) (layer "F.SilkS"))
  (fp_line (start 1 -3) (end -19 -3) (stroke (width 0.2) (type solid)) (layer "F.SilkS"))
  (fp_line (start 1 1) (end 1 -3) (stroke (width 0.2) (type solid)) (layer "F.SilkS"))
  (fp_line (start 1.6 0) (end 1.6 0) (stroke (width 0.1) (type solid)) (layer "F.SilkS"))
  (fp_line (start 1.7 0) (end 1.7 0) (stroke (width 0.1) (type solid)) (layer "F.SilkS"))
  (fp_line (start 1.7 0) (end 1.7 0) (stroke (width 0.1) (type solid)) (layer "F.SilkS"))
  (fp_arc (start 1.6 0) (mid 1.65 -0.05) (end 1.7 0) (stroke (width 0.1) (type solid)) (layer "F.SilkS"))
  (fp_arc (start 1.6 0) (mid 1.65 -0.05) (end 1.7 0) (stroke (width 0.1) (type solid)) (layer "F.SilkS"))
  (fp_arc (start 1.7 0) (mid 1.65 0.05) (end 1.6 0) (stroke (width 0.1) (type solid)) (layer "F.SilkS"))
  (pad "1" thru_hole rect (at 0 0) (size 1.416 1.416) (drill 0.91) (layers "*.Cu" "*.Mask") (remove_unused_layers no)
   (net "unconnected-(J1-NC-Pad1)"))
  (pad "2" thru_hole circle (at 0 -2) (size 1.416 1.416) (drill 0.91) (layers "*.Cu" "*.Mask") (remove_unused_layers no) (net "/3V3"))
  (pad "3" thru_hole circle (at -2 0) (size 1.416 1.416) (drill 0.91) (layers "*.Cu" "*.Mask") (remove_unused_layers no)
   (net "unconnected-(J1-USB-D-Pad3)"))
  (pad "4" thru_hole circle (at -2 -2) (size 1.416 1.416) (drill 0.91) (layers "*.Cu" "*.Mask") (remove_unused_layers no)
   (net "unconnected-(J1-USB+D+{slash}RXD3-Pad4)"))
  (pad "5" thru_hole circle (at -4 0) (size 1.416 1.416) (drill 0.91) (layers "*.Cu" "*.Mask") (remove_unused_layers no)
   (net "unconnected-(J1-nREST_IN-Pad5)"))
  (pad "6" thru_hole circle (at -4 -2) (size 1.416 1.416) (drill 0.91) (layers "*.Cu" "*.Mask") (remove_unused_layers no)
   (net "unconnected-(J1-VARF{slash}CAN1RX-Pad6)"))
  (pad "7" thru_hole circle (at -6 0) (size 1.416 1.416) (drill 0.91) (layers "*.Cu" "*.Mask") (remove_unused_layers no)
   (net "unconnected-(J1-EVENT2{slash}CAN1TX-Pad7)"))
  (pad "8" thru_hole circle (at -6 -2) (size 1.416 1.416) (drill 0.91) (layers "*.Cu" "*.Mask") (remove_unused_layers no)
   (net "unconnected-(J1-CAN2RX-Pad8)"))
  (pad "9" thru_hole circle (at -8 0) (size 1.416 1.416) (drill 0.91) (layers "*.Cu" "*.Mask") (remove_unused_layers no)
   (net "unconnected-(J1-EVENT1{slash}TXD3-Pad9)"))
  (pad "10" thru_hole circle (at -8 -2) (size 1.416 1.416) (drill 0.91) (layers "*.Cu" "*.Mask") (remove_unused_layers no) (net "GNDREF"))
  (pad "11" thru_hole circle (at -10 0) (size 1.416 1.416) (drill 0.91) (layers "*.Cu" "*.Mask") (remove_unused_layers no) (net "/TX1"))
  (pad "12" thru_hole circle (at -10 -2) (size 1.416 1.416) (drill 0.91) (layers "*.Cu" "*.Mask") (remove_unused_layers no) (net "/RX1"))
  (pad "13" thru_hole circle (at -12 0) (size 1.416 1.416) (drill 0.91) (layers "*.Cu" "*.Mask") (remove_unused_layers no) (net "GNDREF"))
  (pad "14" thru_hole circle (at -12 -2) (size 1.416 1.416) (drill 0.91) (layers "*.Cu" "*.Mask") (remove_unused_layers no)
   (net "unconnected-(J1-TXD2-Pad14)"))
  (pad "15" thru_hole circle (at -14 0) (size 1.416 1.416) (drill 0.91) (layers "*.Cu" "*.Mask") (remove_unused_layers no)
   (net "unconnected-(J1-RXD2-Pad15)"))
  (pad "16" thru_hole circle (at -14 -2) (size 1.416 1.416) (drill 0.91) (layers "*.Cu" "*.Mask") (remove_unused_layers no) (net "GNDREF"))
  (pad "17" thru_hole circle (at -16 0) (size 1.416 1.416) (drill 0.91) (layers "*.Cu" "*.Mask") (remove_unused_layers no)
   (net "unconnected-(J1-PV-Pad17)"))
  (pad "18" thru_hole circle (at -16 -2) (size 1.416 1.416) (drill 0.91) (layers "*.Cu" "*.Mask") (remove_unused_layers no) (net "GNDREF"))
  (pad "19" thru_hole circle (at -18 0) (size 1.416 1.416) (drill 0.91) (layers "*.Cu" "*.Mask") (remove_unused_layers no)
   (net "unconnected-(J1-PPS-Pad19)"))
  (pad "20" thru_hole circle (at -18 -2) (size 1.416 1.416) (drill 0.91) (layers "*.Cu" "*.Mask") (remove_unused_layers no)
   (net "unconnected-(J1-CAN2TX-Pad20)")))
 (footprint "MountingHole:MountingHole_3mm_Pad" (layer "F.Cu") (at 189.587 139.421 180)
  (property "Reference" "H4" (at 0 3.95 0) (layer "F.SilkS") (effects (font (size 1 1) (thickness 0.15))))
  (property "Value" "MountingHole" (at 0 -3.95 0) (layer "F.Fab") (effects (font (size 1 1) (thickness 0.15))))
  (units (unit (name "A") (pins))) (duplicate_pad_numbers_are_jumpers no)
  (pad "1" thru_hole circle (at 0 0 180) (size 6 6) (drill 3) (layers "*.Cu" "*.Mask") (remove_unused_layers no) (zone_connect 2)))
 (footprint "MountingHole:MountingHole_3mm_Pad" (layer "F.Cu") (at 166.9 137.025)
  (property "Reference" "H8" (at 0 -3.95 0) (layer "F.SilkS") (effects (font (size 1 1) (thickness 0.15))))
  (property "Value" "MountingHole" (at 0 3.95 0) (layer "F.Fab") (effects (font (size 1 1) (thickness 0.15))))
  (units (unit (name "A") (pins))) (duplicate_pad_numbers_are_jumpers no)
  (pad "1" thru_hole circle (at 0 0) (size 6 6) (drill 3) (layers "*.Cu" "*.Mask") (remove_unused_layers no) (zone_connect 2)))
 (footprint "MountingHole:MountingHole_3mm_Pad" (layer "F.Cu") (at 113.411638 53.751219 180)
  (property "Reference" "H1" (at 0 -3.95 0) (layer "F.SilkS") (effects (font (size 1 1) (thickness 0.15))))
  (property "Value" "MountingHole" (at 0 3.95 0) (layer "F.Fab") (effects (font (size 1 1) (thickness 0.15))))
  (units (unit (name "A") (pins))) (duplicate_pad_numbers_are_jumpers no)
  (pad "1" thru_hole circle (at 0 0 180) (size 6 6) (drill 3) (layers "*.Cu" "*.Mask") (remove_unused_layers no) (zone_connect 2)))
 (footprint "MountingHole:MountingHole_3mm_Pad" (layer "F.Cu") (at 132.61 72.255)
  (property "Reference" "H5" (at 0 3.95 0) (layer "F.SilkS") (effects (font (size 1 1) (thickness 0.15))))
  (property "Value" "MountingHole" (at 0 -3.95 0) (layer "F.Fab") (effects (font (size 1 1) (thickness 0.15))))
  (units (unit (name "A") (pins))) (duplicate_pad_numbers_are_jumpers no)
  (pad "1" thru_hole circle (at 0 0) (size 6 6) (drill 3) (layers "*.Cu" "*.Mask") (remove_unused_layers no) (zone_connect 2)))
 (gr_circle (center 157.53 135.755) (end 161.3 135.9) (stroke (width 0.1) (type solid)) (fill no) (layer "F.SilkS"))
 (gr_line (start 105.45961 68.879186) (end 105.45961 50.54279) (stroke (width 0.05) (type default)) (layer "Edge.Cuts"))
 (gr_line (start 105.45961 68.879186) (end 105.4604 138.7468) (stroke (width 0.05) (type solid)) (layer "Edge.Cuts"))
 (gr_line (start 105.4604 142.66989) (end 105.4604 138.7468) (stroke (width 0.05) (type default)) (layer "Edge.Cuts"))
 (gr_line (start 109.45 142.66989) (end 105.4604 142.66989) (stroke (width 0.05) (type default)) (layer "Edge.Cuts"))
 (gr_line (start 109.45 142.66989) (end 189.612 142.67338) (stroke (width 0.05) (type solid)) (layer "Edge.Cuts"))
 (gr_line (start 113.3345 50.54279) (end 105.45961 50.54279) (stroke (width 0.05) (type default)) (layer "Edge.Cuts"))
 (gr_rect (start 136.36 130.65) (end 163.15 140.85) (radius 1) (stroke (width 0.05) (type solid)) (fill no) (layer "Edge.Cuts"))
 (gr_line (start 186.95 50.536244) (end 113.3345 50.54279) (stroke (width 0.05) (type solid)) (layer "Edge.Cuts"))
 (gr_line (start 186.95 50.536244) (end 194.59355 50.536244) (stroke (width 0.05) (type default)) (layer "Edge.Cuts"))
 (gr_line (start 189.61302 142.673376) (end 194.593554 142.673376) (stroke (width 0.05) (type default)) (layer "Edge.Cuts"))
 (gr_line (start 194.59355 68.47) (end 194.59355 50.536244) (stroke (width 0.05) (type default)) (layer "Edge.Cuts"))
 (gr_line (start 194.59355 133.821) (end 194.59355 68.47) (stroke (width 0.05) (type solid)) (layer "Edge.Cuts"))
 (gr_line (start 194.593554 133.820261) (end 194.593554 142.673376) (stroke (width 0.05) (type default)) (layer "Edge.Cuts"))
 (segment (start 171.446638 61.792819) (end 171.863438 61.376019) (width 0.254) (layer "F.Cu") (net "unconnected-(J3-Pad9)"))
 (segment (start 169.303438 61.756019) (end 169.503438 61.556019) (width 0.254) (layer "F.Cu") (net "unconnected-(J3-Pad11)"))
 (segment (start 169.503438 61.556019) (end 169.323438 61.376019) (width 0.254) (layer "F.Cu") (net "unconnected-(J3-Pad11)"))
 (segment (start 166.578438 61.691679) (end 166.783438 61.486679) (width 0.254) (layer "F.Cu") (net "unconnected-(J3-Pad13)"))
 (segment (start 166.783438 61.486679) (end 166.783438 61.376019) (width 0.254) (layer "F.Cu") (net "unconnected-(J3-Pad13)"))
 (segment (start 164.583438 61.376019) (end 164.243438 61.376019) (width 0.254) (layer "F.Cu") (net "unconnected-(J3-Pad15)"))
 (segment (start 143.923438 61.516879) (end 143.923438 61.376019) (width 0.254) (layer "F.Cu") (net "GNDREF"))
 (segment (start 143.923438 53.756019) (end 143.643438 53.756019) (width 0.254) (layer "F.Cu") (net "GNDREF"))
 (segment (start 131.206138 61.393319) (end 131.223438 61.376019) (width 0.254) (layer "F.Cu") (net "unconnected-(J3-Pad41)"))
 (segment (start 141.383438 53.756019) (end 140.843438 53.756019) (width 0.254) (layer "F.Cu") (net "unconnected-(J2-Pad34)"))
 (segment (start 138.843438 53.756019) (end 138.443438 53.756019) (width 0.254) (layer "F.Cu") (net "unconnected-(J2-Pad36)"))
 (segment (start 133.763438 53.756019) (end 133.763438 53.061019) (width 0.254) (layer "F.Cu") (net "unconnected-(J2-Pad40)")))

